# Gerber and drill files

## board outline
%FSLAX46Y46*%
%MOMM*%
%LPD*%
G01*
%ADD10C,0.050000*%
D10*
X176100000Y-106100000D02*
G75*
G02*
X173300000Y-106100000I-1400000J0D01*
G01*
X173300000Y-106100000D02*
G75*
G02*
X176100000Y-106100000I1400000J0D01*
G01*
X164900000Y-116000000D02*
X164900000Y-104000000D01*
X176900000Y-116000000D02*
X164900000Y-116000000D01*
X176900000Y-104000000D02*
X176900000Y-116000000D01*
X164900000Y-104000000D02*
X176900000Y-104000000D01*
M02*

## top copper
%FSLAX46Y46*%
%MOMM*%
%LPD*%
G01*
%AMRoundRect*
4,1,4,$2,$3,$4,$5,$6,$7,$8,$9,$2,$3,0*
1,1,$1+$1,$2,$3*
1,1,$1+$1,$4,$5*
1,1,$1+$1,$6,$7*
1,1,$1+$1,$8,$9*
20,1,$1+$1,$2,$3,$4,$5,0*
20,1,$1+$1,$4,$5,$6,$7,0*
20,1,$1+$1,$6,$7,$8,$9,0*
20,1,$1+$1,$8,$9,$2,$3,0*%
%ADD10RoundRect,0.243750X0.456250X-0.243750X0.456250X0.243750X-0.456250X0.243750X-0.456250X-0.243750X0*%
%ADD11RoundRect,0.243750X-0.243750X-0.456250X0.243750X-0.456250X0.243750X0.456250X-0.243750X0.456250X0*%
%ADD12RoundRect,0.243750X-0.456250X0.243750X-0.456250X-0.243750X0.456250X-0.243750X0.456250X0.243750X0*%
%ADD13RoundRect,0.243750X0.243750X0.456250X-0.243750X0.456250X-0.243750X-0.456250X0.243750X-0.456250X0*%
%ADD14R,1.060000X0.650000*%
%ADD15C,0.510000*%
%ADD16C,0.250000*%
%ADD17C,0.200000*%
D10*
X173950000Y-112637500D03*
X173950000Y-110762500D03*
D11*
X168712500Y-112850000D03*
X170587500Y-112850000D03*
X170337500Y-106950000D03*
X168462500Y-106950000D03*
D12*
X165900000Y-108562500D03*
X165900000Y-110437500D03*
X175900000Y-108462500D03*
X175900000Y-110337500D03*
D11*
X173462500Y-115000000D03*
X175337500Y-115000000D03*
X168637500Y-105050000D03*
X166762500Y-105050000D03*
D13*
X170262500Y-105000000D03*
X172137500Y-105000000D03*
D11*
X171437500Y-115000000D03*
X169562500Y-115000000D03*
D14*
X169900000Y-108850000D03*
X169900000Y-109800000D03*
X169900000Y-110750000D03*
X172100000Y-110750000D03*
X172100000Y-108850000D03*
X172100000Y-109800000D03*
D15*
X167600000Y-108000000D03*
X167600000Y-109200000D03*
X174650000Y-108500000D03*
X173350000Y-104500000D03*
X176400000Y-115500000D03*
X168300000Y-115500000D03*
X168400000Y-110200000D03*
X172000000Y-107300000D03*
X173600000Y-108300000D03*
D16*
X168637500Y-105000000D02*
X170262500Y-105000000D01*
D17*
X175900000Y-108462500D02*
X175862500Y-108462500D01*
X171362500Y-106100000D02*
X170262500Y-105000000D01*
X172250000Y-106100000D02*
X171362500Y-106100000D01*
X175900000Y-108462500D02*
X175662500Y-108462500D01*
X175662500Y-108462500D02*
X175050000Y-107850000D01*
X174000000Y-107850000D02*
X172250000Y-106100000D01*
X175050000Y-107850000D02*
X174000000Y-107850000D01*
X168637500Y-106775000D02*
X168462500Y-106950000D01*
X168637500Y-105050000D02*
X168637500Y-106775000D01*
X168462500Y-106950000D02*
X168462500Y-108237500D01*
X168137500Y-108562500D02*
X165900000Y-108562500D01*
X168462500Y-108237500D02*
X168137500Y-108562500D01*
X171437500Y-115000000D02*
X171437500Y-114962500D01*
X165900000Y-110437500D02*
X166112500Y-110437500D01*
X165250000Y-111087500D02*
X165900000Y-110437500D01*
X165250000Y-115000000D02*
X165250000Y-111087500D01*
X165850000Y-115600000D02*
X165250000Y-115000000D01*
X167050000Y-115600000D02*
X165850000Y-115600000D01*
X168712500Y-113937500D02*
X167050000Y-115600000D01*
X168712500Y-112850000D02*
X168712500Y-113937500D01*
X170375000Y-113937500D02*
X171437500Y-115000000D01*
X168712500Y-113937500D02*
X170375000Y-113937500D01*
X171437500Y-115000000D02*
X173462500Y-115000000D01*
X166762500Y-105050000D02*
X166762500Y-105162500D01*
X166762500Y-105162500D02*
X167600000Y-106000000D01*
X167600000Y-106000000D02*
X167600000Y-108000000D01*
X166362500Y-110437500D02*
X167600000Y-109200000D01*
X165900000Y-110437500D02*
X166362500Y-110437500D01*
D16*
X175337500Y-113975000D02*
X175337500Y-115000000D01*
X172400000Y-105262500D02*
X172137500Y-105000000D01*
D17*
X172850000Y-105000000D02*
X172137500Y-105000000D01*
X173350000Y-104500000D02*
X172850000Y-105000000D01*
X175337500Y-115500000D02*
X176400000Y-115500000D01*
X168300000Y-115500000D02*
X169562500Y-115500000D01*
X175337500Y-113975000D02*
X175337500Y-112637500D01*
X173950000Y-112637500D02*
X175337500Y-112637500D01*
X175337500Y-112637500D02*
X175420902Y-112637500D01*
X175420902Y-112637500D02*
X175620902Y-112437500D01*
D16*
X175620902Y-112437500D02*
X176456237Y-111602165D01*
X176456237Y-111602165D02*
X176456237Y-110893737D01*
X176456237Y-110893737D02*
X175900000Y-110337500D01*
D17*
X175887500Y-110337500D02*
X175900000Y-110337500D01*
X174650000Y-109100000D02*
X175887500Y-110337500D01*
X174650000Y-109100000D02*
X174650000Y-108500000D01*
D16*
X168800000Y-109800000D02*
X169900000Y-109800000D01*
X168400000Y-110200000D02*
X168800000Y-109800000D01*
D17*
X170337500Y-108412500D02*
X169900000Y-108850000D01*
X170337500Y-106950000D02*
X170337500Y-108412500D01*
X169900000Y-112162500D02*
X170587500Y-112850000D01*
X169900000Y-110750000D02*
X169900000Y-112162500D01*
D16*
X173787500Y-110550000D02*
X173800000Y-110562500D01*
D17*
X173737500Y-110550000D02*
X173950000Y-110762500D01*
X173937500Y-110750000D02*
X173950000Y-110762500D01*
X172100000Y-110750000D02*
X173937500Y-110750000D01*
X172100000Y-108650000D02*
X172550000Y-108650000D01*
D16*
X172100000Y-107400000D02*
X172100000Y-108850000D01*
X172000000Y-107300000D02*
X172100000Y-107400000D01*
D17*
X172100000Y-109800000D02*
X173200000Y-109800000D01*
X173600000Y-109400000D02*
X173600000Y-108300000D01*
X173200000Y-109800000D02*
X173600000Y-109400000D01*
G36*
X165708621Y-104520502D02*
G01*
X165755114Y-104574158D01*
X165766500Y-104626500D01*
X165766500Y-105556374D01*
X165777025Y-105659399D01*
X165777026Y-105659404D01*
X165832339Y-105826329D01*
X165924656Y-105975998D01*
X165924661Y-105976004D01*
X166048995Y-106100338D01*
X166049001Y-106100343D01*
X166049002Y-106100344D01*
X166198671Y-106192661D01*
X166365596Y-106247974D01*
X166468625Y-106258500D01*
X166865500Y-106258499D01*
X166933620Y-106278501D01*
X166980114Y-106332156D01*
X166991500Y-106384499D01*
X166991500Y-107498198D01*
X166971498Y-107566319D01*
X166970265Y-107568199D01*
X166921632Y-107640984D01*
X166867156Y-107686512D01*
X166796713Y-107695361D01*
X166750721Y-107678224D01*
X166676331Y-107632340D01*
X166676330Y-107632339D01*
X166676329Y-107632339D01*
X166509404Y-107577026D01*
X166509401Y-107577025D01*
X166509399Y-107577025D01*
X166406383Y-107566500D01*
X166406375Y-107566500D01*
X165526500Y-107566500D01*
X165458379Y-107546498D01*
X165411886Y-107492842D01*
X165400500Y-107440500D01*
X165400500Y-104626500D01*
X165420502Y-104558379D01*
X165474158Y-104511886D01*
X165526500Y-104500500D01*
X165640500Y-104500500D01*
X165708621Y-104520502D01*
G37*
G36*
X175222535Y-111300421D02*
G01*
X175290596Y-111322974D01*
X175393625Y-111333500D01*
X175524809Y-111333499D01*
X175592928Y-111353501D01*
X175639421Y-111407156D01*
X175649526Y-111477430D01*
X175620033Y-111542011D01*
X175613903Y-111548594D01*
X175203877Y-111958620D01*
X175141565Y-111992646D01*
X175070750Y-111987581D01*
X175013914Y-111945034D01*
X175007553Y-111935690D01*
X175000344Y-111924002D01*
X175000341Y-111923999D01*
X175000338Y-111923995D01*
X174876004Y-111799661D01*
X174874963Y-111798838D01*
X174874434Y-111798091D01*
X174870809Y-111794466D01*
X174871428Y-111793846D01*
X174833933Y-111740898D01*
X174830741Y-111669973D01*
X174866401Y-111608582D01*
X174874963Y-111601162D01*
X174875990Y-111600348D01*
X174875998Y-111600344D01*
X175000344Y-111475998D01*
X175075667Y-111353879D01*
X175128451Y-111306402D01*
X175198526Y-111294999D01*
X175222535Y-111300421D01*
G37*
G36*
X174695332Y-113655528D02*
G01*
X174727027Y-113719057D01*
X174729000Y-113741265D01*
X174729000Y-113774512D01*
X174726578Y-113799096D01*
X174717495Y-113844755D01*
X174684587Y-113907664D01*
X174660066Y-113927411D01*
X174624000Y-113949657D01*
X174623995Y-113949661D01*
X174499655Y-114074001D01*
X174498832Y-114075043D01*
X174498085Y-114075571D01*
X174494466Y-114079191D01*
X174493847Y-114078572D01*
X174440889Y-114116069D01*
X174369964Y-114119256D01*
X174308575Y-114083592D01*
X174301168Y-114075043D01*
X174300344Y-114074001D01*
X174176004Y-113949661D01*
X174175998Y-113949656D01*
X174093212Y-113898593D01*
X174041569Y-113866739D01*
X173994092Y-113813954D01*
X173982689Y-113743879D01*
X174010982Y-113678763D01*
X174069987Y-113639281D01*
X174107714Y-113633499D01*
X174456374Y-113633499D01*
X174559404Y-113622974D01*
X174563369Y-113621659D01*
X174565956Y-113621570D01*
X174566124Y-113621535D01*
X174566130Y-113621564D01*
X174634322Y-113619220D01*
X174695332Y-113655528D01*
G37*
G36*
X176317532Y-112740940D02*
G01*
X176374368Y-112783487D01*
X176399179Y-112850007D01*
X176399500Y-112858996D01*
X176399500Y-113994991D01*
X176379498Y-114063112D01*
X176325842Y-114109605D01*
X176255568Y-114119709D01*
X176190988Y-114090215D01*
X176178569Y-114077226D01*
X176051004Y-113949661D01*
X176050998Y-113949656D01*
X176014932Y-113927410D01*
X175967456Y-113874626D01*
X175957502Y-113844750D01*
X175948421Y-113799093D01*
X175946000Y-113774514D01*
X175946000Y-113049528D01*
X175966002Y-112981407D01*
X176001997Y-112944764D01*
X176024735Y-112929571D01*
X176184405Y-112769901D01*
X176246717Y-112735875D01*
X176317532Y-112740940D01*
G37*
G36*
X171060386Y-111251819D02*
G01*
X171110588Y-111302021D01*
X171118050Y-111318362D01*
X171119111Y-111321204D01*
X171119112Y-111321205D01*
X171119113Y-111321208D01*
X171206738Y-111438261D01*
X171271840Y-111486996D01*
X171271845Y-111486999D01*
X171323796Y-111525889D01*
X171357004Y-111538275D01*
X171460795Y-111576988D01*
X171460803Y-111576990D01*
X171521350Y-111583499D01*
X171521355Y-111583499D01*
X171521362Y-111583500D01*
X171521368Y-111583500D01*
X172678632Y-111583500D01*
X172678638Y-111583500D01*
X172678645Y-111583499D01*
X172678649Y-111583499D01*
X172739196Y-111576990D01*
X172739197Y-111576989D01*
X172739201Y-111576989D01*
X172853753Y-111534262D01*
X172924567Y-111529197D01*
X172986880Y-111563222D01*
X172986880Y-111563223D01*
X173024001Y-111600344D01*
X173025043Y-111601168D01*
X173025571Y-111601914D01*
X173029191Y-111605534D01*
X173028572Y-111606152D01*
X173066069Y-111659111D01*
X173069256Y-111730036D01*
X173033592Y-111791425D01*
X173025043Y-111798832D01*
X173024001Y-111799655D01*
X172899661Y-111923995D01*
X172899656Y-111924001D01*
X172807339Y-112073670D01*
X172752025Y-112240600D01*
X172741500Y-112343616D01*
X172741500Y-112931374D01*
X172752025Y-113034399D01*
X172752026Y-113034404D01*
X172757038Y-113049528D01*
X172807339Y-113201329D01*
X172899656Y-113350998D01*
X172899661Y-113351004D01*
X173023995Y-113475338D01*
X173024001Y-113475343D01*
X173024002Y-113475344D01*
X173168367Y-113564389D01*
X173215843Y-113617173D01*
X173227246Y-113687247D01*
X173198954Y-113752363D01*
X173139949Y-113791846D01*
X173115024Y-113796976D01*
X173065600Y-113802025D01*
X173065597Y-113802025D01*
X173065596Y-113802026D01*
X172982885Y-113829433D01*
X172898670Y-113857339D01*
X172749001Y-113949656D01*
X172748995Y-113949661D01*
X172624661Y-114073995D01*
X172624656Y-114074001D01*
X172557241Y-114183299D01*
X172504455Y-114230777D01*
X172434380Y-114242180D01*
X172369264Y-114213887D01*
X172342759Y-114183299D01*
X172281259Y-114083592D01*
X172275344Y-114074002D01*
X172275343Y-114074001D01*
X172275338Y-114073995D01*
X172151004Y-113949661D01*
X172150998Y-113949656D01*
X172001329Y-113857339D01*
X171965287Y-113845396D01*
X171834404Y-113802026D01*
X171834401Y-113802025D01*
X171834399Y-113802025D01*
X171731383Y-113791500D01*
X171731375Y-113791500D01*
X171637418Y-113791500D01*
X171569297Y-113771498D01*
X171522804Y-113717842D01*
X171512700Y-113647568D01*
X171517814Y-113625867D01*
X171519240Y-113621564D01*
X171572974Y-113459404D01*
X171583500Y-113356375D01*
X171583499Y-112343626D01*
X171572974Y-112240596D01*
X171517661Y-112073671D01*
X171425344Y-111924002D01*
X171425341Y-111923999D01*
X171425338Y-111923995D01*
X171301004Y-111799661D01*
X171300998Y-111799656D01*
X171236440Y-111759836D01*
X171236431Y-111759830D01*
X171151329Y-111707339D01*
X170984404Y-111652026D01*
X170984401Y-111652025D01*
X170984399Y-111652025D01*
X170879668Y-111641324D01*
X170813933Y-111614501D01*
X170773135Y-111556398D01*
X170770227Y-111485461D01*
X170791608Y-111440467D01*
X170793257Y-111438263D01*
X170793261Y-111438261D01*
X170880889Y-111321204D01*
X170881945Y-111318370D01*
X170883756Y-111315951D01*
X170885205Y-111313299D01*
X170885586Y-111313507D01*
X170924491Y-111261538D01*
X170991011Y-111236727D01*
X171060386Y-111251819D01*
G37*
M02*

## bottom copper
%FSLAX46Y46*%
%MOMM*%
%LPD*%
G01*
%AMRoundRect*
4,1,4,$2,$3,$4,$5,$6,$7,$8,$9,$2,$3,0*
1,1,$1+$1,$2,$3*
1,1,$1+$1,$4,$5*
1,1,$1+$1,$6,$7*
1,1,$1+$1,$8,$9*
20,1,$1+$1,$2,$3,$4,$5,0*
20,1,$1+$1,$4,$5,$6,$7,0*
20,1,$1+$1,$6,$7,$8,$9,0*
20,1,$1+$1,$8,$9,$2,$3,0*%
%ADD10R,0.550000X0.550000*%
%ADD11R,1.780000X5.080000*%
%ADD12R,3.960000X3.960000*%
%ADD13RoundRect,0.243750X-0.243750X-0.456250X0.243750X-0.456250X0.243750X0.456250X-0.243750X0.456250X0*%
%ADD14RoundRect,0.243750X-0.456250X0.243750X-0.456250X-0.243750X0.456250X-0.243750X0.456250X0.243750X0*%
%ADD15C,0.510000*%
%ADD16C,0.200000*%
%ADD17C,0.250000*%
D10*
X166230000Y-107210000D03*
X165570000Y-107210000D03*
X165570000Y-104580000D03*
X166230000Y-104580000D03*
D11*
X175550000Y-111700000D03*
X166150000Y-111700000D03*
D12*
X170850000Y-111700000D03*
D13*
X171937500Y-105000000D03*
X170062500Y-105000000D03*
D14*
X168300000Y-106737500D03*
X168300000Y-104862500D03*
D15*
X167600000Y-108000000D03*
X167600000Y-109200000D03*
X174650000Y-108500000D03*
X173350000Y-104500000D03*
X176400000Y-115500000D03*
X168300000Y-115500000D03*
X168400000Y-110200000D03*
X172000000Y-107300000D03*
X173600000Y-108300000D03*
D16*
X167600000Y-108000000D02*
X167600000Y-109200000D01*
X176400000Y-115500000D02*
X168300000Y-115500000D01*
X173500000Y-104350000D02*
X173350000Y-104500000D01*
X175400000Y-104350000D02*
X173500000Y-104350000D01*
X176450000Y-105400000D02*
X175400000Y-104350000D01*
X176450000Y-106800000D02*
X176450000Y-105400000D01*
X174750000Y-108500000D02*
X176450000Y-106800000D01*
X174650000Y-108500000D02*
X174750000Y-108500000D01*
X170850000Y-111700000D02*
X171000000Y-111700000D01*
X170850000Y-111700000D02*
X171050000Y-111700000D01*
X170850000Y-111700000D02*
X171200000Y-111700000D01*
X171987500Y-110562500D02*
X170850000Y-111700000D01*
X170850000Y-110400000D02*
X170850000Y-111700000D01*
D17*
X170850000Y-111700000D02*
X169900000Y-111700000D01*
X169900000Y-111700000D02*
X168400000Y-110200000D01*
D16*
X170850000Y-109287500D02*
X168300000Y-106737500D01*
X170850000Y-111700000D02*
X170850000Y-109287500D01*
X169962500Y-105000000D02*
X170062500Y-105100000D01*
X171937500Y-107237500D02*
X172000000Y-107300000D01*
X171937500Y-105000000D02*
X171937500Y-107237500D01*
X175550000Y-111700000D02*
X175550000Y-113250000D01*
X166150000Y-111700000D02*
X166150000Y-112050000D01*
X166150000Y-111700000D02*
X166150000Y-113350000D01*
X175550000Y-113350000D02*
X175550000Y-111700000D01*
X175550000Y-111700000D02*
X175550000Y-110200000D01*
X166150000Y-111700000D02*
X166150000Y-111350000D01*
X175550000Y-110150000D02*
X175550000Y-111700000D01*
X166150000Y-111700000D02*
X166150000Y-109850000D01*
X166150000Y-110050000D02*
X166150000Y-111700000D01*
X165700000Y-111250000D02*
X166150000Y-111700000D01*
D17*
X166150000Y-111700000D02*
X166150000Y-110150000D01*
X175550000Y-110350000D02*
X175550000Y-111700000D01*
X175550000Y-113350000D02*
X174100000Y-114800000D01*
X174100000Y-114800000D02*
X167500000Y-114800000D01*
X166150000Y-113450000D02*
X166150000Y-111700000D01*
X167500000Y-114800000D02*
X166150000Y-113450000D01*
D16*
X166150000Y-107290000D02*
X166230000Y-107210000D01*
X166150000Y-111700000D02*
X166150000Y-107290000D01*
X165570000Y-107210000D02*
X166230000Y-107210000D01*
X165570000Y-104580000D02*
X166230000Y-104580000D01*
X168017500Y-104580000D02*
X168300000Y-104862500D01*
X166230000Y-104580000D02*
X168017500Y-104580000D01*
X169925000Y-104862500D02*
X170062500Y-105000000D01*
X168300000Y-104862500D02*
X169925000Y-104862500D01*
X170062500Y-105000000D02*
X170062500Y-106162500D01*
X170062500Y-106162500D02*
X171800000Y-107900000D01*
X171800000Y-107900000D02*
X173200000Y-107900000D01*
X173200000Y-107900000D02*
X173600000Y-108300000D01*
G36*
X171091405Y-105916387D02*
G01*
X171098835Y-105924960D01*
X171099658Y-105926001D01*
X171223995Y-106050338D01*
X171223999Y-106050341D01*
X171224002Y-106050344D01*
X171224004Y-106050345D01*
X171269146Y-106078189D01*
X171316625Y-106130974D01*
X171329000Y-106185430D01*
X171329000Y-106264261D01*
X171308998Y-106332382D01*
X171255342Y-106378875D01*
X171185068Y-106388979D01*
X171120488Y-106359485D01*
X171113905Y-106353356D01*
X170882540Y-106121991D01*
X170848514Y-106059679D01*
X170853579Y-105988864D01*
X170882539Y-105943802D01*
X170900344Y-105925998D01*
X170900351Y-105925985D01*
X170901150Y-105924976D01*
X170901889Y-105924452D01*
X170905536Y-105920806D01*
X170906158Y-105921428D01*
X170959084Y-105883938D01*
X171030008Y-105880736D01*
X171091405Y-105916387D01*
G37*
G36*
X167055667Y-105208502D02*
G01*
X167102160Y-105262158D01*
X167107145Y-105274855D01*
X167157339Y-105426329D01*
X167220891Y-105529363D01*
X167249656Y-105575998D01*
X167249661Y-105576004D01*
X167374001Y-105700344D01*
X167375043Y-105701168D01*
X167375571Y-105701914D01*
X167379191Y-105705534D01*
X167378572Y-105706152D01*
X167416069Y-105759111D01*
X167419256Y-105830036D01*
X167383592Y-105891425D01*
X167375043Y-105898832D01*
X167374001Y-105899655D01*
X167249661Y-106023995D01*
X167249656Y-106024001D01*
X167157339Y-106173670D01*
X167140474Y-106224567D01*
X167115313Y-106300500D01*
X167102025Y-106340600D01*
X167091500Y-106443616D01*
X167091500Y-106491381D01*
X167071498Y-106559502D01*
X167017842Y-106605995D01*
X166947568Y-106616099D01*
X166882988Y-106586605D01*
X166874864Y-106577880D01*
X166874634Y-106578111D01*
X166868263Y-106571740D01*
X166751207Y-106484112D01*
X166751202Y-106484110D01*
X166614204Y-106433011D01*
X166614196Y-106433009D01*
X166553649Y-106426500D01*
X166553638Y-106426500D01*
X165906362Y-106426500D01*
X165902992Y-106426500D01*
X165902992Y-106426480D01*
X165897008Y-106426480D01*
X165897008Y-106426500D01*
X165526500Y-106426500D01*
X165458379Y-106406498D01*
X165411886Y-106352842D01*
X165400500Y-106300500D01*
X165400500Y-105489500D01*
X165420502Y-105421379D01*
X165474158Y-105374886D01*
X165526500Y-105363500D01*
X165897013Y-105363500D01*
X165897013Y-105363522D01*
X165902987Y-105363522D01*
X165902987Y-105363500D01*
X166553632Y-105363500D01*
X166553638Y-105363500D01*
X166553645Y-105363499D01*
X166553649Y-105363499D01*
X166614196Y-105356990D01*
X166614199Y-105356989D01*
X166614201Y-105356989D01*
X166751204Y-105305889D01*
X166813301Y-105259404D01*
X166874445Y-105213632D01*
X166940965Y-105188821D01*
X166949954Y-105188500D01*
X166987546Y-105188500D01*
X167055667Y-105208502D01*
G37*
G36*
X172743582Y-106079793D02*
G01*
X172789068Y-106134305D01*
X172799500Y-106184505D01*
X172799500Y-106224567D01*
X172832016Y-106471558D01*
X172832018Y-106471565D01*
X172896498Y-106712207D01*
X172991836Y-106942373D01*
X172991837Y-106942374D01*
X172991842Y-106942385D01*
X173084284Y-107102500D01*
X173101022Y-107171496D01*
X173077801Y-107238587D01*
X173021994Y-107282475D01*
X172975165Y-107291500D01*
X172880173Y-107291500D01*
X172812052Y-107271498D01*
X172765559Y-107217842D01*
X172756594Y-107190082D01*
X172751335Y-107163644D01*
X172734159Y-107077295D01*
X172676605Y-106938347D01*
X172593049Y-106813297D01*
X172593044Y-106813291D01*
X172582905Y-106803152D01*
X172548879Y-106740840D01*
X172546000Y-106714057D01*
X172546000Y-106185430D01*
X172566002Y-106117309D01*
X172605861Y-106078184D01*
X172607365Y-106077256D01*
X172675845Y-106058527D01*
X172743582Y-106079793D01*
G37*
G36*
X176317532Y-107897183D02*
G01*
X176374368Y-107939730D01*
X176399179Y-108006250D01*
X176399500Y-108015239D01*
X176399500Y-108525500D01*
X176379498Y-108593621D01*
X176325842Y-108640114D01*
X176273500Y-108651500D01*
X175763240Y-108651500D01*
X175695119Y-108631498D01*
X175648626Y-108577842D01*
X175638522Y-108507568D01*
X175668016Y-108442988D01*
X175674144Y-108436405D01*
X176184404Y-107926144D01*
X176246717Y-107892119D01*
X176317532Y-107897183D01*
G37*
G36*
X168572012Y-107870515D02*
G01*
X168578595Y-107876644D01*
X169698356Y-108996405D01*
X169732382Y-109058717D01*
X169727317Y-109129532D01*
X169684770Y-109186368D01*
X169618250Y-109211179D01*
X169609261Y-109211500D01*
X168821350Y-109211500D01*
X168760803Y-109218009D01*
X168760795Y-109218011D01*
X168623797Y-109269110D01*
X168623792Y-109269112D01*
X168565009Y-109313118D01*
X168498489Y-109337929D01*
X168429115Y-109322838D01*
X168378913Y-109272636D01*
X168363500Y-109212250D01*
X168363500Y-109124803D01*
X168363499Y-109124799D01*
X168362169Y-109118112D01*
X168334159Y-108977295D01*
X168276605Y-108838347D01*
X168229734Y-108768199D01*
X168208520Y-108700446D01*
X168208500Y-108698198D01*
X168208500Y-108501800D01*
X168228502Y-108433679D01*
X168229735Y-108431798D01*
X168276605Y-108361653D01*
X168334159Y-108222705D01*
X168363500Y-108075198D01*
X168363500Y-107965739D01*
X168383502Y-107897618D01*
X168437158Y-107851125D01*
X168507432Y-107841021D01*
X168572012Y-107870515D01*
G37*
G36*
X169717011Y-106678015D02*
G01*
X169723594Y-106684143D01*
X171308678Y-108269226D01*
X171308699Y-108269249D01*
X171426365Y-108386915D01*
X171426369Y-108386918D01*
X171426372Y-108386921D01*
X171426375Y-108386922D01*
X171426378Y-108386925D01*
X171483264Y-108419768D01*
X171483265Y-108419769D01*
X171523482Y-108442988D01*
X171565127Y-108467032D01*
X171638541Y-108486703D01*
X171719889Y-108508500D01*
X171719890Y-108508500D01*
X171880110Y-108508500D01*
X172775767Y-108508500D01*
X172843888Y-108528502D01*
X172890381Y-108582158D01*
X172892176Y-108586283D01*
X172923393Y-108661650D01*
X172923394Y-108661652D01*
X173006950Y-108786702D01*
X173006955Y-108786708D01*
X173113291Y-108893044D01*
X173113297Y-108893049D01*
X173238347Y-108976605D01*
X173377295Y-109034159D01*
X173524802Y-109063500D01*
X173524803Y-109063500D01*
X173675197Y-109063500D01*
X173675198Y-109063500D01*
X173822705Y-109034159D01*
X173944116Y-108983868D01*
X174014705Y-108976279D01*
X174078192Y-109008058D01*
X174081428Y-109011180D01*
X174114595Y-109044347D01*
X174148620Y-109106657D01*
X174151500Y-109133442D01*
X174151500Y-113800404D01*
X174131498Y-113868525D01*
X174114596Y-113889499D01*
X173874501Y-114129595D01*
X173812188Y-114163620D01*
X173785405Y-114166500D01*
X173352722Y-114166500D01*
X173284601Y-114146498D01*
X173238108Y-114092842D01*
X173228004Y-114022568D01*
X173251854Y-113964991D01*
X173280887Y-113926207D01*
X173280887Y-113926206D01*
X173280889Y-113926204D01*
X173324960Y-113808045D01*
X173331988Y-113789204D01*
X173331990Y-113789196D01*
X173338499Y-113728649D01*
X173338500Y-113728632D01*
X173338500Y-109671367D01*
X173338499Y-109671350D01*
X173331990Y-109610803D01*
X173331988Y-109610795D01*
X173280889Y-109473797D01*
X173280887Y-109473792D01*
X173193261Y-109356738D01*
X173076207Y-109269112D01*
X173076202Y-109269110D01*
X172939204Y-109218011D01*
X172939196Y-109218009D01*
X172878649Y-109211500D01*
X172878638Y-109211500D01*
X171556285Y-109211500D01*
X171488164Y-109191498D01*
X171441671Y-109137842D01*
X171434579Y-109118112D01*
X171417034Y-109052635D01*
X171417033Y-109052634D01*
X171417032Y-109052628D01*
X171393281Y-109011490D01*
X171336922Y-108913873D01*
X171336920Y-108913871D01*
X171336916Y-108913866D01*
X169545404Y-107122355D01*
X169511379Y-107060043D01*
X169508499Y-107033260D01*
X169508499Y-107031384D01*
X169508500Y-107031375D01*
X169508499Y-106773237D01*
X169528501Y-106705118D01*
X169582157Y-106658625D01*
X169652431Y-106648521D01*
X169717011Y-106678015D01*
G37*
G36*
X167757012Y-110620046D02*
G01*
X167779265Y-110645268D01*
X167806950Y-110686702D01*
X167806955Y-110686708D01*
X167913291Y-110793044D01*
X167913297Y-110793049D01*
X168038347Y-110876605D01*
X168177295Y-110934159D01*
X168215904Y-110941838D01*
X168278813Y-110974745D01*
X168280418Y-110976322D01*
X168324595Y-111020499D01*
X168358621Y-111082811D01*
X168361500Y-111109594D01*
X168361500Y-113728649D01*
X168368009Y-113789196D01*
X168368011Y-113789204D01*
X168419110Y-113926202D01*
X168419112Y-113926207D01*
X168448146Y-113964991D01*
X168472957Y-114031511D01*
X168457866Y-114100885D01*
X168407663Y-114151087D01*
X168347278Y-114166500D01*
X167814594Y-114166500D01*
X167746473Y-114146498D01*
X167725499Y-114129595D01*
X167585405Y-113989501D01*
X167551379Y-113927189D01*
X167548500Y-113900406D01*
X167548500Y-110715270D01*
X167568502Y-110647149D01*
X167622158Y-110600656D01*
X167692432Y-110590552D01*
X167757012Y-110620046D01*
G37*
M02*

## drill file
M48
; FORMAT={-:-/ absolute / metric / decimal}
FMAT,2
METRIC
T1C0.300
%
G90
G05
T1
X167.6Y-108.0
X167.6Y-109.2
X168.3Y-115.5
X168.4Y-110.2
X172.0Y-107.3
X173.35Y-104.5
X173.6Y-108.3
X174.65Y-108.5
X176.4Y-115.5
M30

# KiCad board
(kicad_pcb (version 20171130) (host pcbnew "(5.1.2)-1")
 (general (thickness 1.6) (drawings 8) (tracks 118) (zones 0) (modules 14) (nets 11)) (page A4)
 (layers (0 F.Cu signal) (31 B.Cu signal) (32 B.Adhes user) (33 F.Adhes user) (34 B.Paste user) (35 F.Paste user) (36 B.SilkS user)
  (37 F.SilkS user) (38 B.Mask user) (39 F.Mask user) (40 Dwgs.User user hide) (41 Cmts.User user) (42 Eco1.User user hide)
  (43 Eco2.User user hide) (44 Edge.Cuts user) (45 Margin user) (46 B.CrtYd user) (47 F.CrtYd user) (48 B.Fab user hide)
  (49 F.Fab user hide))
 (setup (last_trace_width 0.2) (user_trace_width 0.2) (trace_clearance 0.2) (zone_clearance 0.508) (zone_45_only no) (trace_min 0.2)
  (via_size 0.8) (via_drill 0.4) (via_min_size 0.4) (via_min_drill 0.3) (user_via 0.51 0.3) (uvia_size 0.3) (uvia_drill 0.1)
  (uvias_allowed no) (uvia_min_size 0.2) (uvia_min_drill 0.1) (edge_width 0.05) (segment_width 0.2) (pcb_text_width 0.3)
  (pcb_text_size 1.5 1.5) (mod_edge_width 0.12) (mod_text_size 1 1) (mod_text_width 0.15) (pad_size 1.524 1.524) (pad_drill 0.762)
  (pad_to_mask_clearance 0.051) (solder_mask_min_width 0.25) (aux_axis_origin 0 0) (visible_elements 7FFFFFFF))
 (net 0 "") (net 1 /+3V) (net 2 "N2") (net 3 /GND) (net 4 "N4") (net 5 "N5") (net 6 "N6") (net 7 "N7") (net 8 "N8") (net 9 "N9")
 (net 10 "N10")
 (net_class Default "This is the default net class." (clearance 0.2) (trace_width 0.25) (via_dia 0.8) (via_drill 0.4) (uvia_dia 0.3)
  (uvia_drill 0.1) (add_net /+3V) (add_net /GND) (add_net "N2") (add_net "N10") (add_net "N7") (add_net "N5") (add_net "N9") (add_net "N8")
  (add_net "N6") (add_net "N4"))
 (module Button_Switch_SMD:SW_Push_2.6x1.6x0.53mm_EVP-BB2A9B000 (layer B.Cu) (at 165.9 105.9 90)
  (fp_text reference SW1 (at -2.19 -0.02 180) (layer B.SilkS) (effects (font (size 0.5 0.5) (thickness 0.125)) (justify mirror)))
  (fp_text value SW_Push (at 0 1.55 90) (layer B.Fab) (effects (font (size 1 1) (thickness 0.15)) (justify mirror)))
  (pad 1 smd rect (at -1.31 0.33 90) (size 0.55 0.55) (layers B.Cu B.Paste B.Mask) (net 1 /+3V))
  (pad 1 smd rect (at -1.31 -0.33 90) (size 0.55 0.55) (layers B.Cu B.Paste B.Mask) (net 1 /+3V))
  (pad 2 smd rect (at 1.32 -0.33 90) (size 0.55 0.55) (layers B.Cu B.Paste B.Mask) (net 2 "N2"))
  (pad 2 smd rect (at 1.32 0.33 90) (size 0.55 0.55) (layers B.Cu B.Paste B.Mask) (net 2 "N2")))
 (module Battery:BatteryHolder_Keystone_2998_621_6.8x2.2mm (layer B.Cu) (at 170.85 111.7)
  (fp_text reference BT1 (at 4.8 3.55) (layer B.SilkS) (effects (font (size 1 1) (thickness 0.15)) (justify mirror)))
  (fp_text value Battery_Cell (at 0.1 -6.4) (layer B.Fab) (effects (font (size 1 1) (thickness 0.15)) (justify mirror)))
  (pad 1 smd rect (at 4.7 0) (size 1.78 5.08) (layers B.Cu B.Paste B.Mask) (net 1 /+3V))
  (pad 1 smd rect (at -4.7 0) (size 1.78 5.08) (layers B.Cu B.Paste B.Mask) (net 1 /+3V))
  (pad 2 smd rect (at 0 0) (size 3.96 3.96) (layers B.Cu B.Paste B.Mask) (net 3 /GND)))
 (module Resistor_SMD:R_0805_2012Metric (layer B.Cu) (at 171 105)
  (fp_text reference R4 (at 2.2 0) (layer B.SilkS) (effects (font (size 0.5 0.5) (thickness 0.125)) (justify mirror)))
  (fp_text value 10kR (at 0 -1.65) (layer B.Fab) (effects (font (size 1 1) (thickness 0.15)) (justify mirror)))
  (pad 2 smd roundrect (at 0.9375 0) (size 0.975 1.4) (layers B.Cu B.Paste B.Mask) (roundrect_rratio 0.25) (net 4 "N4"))
  (pad 1 smd roundrect (at -0.9375 0) (size 0.975 1.4) (layers B.Cu B.Paste B.Mask) (roundrect_rratio 0.25) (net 2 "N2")))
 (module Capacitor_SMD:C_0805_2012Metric (layer B.Cu) (at 168.3 105.8 270)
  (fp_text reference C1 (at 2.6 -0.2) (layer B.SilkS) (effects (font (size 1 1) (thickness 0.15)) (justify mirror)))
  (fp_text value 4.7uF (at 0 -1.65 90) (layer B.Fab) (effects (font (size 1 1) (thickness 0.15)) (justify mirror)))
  (pad 2 smd roundrect (at 0.9375 0 270) (size 0.975 1.4) (layers B.Cu B.Paste B.Mask) (roundrect_rratio 0.25) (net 3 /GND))
  (pad 1 smd roundrect (at -0.9375 0 270) (size 0.975 1.4) (layers B.Cu B.Paste B.Mask) (roundrect_rratio 0.25) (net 2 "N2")))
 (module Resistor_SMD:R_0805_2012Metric (layer F.Cu) (at 173.95 111.7 90)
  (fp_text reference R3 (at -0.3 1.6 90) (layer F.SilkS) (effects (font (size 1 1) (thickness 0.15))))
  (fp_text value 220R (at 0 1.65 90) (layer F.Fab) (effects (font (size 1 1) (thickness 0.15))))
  (pad 1 smd roundrect (at -0.9375 0 90) (size 0.975 1.4) (layers F.Cu F.Paste F.Mask) (roundrect_rratio 0.25) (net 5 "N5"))
  (pad 2 smd roundrect (at 0.9375 0 90) (size 0.975 1.4) (layers F.Cu F.Paste F.Mask) (roundrect_rratio 0.25) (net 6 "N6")))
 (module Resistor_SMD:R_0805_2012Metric (layer F.Cu) (at 169.65 112.85)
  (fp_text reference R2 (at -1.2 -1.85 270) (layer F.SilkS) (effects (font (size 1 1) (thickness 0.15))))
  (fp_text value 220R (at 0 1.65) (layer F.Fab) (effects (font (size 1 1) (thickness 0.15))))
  (pad 1 smd roundrect (at -0.9375 0) (size 0.975 1.4) (layers F.Cu F.Paste F.Mask) (roundrect_rratio 0.25) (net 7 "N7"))
  (pad 2 smd roundrect (at 0.9375 0) (size 0.975 1.4) (layers F.Cu F.Paste F.Mask) (roundrect_rratio 0.25) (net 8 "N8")))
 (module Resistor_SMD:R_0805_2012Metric (layer F.Cu) (at 169.4 106.95)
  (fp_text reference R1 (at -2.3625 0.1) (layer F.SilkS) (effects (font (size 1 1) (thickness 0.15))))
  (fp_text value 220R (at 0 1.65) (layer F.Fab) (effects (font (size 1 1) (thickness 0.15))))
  (pad 2 smd roundrect (at 0.9375 0) (size 0.975 1.4) (layers F.Cu F.Paste F.Mask) (roundrect_rratio 0.25) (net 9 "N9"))
  (pad 1 smd roundrect (at -0.9375 0) (size 0.975 1.4) (layers F.Cu F.Paste F.Mask) (roundrect_rratio 0.25) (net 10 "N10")))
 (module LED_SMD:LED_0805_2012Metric (layer F.Cu) (at 165.9 109.5 270)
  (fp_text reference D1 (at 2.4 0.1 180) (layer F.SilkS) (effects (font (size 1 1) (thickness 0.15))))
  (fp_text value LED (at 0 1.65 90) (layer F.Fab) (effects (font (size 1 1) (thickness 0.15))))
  (pad 1 smd roundrect (at -0.9375 0 270) (size 0.975 1.4) (layers F.Cu F.Paste F.Mask) (roundrect_rratio 0.25) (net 10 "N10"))
  (pad 2 smd roundrect (at 0.9375 0 270) (size 0.975 1.4) (layers F.Cu F.Paste F.Mask) (roundrect_rratio 0.25) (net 7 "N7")))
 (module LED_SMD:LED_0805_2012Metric (layer F.Cu) (at 175.9 109.4 270)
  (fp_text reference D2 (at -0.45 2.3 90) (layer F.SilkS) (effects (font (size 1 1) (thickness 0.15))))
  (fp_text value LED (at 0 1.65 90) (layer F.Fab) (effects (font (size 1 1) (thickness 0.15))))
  (pad 1 smd roundrect (at -0.9375 0 270) (size 0.975 1.4) (layers F.Cu F.Paste F.Mask) (roundrect_rratio 0.25) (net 10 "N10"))
  (pad 2 smd roundrect (at 0.9375 0 270) (size 0.975 1.4) (layers F.Cu F.Paste F.Mask) (roundrect_rratio 0.25) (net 5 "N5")))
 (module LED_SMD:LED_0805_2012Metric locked (layer F.Cu) (at 174.4 115)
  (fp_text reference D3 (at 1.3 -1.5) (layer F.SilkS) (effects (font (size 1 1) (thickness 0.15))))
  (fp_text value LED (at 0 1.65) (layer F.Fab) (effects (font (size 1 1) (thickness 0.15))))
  (pad 1 smd roundrect (at -0.9375 0) (size 0.975 1.4) (layers F.Cu F.Paste F.Mask) (roundrect_rratio 0.25) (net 7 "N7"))
  (pad 2 smd roundrect (at 0.9375 0) (size 0.975 1.4) (layers F.Cu F.Paste F.Mask) (roundrect_rratio 0.25) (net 5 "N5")))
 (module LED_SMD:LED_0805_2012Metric (layer F.Cu) (at 167.7 105.05)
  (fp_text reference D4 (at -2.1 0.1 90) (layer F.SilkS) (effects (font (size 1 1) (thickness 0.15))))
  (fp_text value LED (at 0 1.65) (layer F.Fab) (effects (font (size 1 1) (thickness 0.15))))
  (pad 2 smd roundrect (at 0.9375 0) (size 0.975 1.4) (layers F.Cu F.Paste F.Mask) (roundrect_rratio 0.25) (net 10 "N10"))
  (pad 1 smd roundrect (at -0.9375 0) (size 0.975 1.4) (layers F.Cu F.Paste F.Mask) (roundrect_rratio 0.25) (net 7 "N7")))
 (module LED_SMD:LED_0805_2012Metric (layer F.Cu) (at 171.2 105 180)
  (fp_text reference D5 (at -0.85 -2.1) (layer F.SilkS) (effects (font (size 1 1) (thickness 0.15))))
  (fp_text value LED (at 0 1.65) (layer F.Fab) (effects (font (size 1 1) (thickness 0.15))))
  (pad 2 smd roundrect (at 0.9375 0 180) (size 0.975 1.4) (layers F.Cu F.Paste F.Mask) (roundrect_rratio 0.25) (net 10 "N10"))
  (pad 1 smd roundrect (at -0.9375 0 180) (size 0.975 1.4) (layers F.Cu F.Paste F.Mask) (roundrect_rratio 0.25) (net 5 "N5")))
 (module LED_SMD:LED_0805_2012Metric (layer F.Cu) (at 170.5 115)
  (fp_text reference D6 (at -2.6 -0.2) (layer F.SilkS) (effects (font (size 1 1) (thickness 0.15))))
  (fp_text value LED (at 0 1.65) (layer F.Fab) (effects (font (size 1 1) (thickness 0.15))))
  (pad 2 smd roundrect (at 0.9375 0) (size 0.975 1.4) (layers F.Cu F.Paste F.Mask) (roundrect_rratio 0.25) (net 7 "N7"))
  (pad 1 smd roundrect (at -0.9375 0) (size 0.975 1.4) (layers F.Cu F.Paste F.Mask) (roundrect_rratio 0.25) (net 5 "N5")))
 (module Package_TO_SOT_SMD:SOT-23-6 (layer F.Cu) (at 171 109.8)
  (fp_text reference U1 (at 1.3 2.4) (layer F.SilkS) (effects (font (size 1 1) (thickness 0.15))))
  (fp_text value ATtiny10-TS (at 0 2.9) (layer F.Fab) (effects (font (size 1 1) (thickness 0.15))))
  (pad 1 smd rect (at -1.1 -0.95) (size 1.06 0.65) (layers F.Cu F.Paste F.Mask) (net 9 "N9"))
  (pad 2 smd rect (at -1.1 0) (size 1.06 0.65) (layers F.Cu F.Paste F.Mask) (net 3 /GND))
  (pad 3 smd rect (at -1.1 0.95) (size 1.06 0.65) (layers F.Cu F.Paste F.Mask) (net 8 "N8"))
  (pad 4 smd rect (at 1.1 0.95) (size 1.06 0.65) (layers F.Cu F.Paste F.Mask) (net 6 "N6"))
  (pad 6 smd rect (at 1.1 -0.95) (size 1.06 0.65) (layers F.Cu F.Paste F.Mask) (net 4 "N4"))
  (pad 5 smd rect (at 1.1 0) (size 1.06 0.65) (layers F.Cu F.Paste F.Mask) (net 2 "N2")))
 (gr_circle (center 174.7 106.1) (end 176.1 106.1) (layer Edge.Cuts) (width 0.05))
 (gr_line (start 164.9 116) (end 164.9 104) (layer Edge.Cuts) (width 0.05))
 (gr_line (start 176.9 116) (end 164.9 116) (layer Edge.Cuts) (width 0.05))
 (gr_line (start 176.9 104) (end 176.9 116) (layer Edge.Cuts) (width 0.05))
 (gr_line (start 164.9 104) (end 176.9 104) (layer Edge.Cuts) (width 0.05))
 (segment (start 168.6375 105) (end 170.2625 105) (width 0.25) (layer F.Cu) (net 10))
 (segment (start 175.9 108.4625) (end 175.8625 108.4625) (width 0.2) (layer F.Cu) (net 10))
 (segment (start 171.3625 106.1) (end 170.2625 105) (width 0.2) (layer F.Cu) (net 10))
 (segment (start 172.25 106.1) (end 171.3625 106.1) (width 0.2) (layer F.Cu) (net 10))
 (segment (start 175.9 108.4625) (end 175.6625 108.4625) (width 0.2) (layer F.Cu) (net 10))
 (segment (start 175.6625 108.4625) (end 175.05 107.85) (width 0.2) (layer F.Cu) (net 10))
 (segment (start 174 107.85) (end 172.25 106.1) (width 0.2) (layer F.Cu) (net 10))
 (segment (start 175.05 107.85) (end 174 107.85) (width 0.2) (layer F.Cu) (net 10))
 (segment (start 168.6375 106.775) (end 168.4625 106.95) (width 0.2) (layer F.Cu) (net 10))
 (segment (start 168.6375 105.05) (end 168.6375 106.775) (width 0.2) (layer F.Cu) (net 10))
 (segment (start 168.4625 106.95) (end 168.4625 108.2375) (width 0.2) (layer F.Cu) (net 10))
 (segment (start 168.1375 108.5625) (end 165.9 108.5625) (width 0.2) (layer F.Cu) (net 10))
 (segment (start 168.4625 108.2375) (end 168.1375 108.5625) (width 0.2) (layer F.Cu) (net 10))
 (segment (start 171.4375 115) (end 171.4375 114.9625) (width 0.2) (layer F.Cu) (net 7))
 (segment (start 165.9 110.4375) (end 166.1125 110.4375) (width 0.2) (layer F.Cu) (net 7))
 (segment (start 165.25 111.0875) (end 165.9 110.4375) (width 0.2) (layer F.Cu) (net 7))
 (segment (start 165.25 115) (end 165.25 111.0875) (width 0.2) (layer F.Cu) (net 7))
 (segment (start 165.85 115.6) (end 165.25 115) (width 0.2) (layer F.Cu) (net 7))
 (segment (start 167.05 115.6) (end 165.85 115.6) (width 0.2) (layer F.Cu) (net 7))
 (segment (start 168.7125 113.9375) (end 167.05 115.6) (width 0.2) (layer F.Cu) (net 7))
 (segment (start 168.7125 112.85) (end 168.7125 113.9375) (width 0.2) (layer F.Cu) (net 7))
 (segment (start 170.375 113.9375) (end 171.4375 115) (width 0.2) (layer F.Cu) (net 7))
 (segment (start 168.7125 113.9375) (end 170.375 113.9375) (width 0.2) (layer F.Cu) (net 7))
 (segment (start 171.4375 115) (end 173.4625 115) (width 0.2) (layer F.Cu) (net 7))
 (segment (start 166.7625 105.05) (end 166.7625 105.1625) (width 0.2) (layer F.Cu) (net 7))
 (via (at 167.6 108) (size 0.51) (drill 0.3) (layers F.Cu B.Cu) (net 7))
 (segment (start 166.7625 105.1625) (end 167.6 106) (width 0.2) (layer F.Cu) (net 7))
 (segment (start 167.6 106) (end 167.6 108) (width 0.2) (layer F.Cu) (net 7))
 (via (at 167.6 109.2) (size 0.51) (drill 0.3) (layers F.Cu B.Cu) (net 7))
 (segment (start 167.6 108) (end 167.6 109.2) (width 0.2) (layer B.Cu) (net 7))
 (segment (start 166.3625 110.4375) (end 167.6 109.2) (width 0.2) (layer F.Cu) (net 7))
 (segment (start 165.9 110.4375) (end 166.3625 110.4375) (width 0.2) (layer F.Cu) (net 7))
 (segment (start 175.3375 113.975) (end 175.3375 115) (width 0.25) (layer F.Cu) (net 5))
 (via (at 174.65 108.5) (size 0.51) (drill 0.3) (layers F.Cu B.Cu) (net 5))
 (segment (start 172.4 105.2625) (end 172.1375 105) (width 0.25) (layer F.Cu) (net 5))
 (via (at 173.35 104.5) (size 0.51) (drill 0.3) (layers F.Cu B.Cu) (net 5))
 (segment (start 172.85 105) (end 172.1375 105) (width 0.2) (layer F.Cu) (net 5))
 (segment (start 173.35 104.5) (end 172.85 105) (width 0.2) (layer F.Cu) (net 5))
 (via (at 176.4 115.5) (size 0.51) (drill 0.3) (layers F.Cu B.Cu) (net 5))
 (segment (start 175.3375 115.5) (end 176.4 115.5) (width 0.2) (layer F.Cu) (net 5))
 (via (at 168.3 115.5) (size 0.51) (drill 0.3) (layers F.Cu B.Cu) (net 5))
 (segment (start 176.4 115.5) (end 168.3 115.5) (width 0.2) (layer B.Cu) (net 5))
 (segment (start 168.3 115.5) (end 169.5625 115.5) (width 0.2) (layer F.Cu) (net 5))
 (segment (start 175.3375 113.975) (end 175.3375 112.6375) (width 0.2) (layer F.Cu) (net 5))
 (segment (start 173.95 112.6375) (end 175.3375 112.6375) (width 0.2) (layer F.Cu) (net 5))
 (segment (start 175.3375 112.6375) (end 175.420902 112.6375) (width 0.2) (layer F.Cu) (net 5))
 (segment (start 175.420902 112.6375) (end 175.620902 112.4375) (width 0.2) (layer F.Cu) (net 5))
 (segment (start 175.620902 112.4375) (end 176.456237 111.602165) (width 0.25) (layer F.Cu) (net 5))
 (segment (start 176.456237 111.602165) (end 176.456237 110.893737) (width 0.25) (layer F.Cu) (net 5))
 (segment (start 176.456237 110.893737) (end 175.9 110.3375) (width 0.25) (layer F.Cu) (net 5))
 (segment (start 173.5 104.35) (end 173.35 104.5) (width 0.2) (layer B.Cu) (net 5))
 (segment (start 175.4 104.35) (end 173.5 104.35) (width 0.2) (layer B.Cu) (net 5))
 (segment (start 176.45 105.4) (end 175.4 104.35) (width 0.2) (layer B.Cu) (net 5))
 (segment (start 176.45 106.8) (end 176.45 105.4) (width 0.2) (layer B.Cu) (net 5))
 (segment (start 175.8875 110.3375) (end 175.9 110.3375) (width 0.2) (layer F.Cu) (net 5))
 (segment (start 174.65 109.1) (end 175.8875 110.3375) (width 0.2) (layer F.Cu) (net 5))
 (segment (start 174.65 109.1) (end 174.65 108.5) (width 0.2) (layer F.Cu) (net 5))
 (segment (start 174.75 108.5) (end 176.45 106.8) (width 0.2) (layer B.Cu) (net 5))
 (segment (start 174.65 108.5) (end 174.75 108.5) (width 0.2) (layer B.Cu) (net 5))
 (segment (start 170.85 111.7) (end 171 111.7) (width 0.2) (layer B.Cu) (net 3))
 (segment (start 170.85 111.7) (end 171.05 111.7) (width 0.2) (layer B.Cu) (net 3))
 (segment (start 170.85 111.7) (end 171.2 111.7) (width 0.2) (layer B.Cu) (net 3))
 (segment (start 171.9875 110.5625) (end 170.85 111.7) (width 0.2) (layer B.Cu) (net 3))
 (segment (start 170.85 110.4) (end 170.85 111.7) (width 0.2) (layer B.Cu) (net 3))
 (via (at 168.4 110.2) (size 0.51) (drill 0.3) (layers F.Cu B.Cu) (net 3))
 (segment (start 170.85 111.7) (end 169.9 111.7) (width 0.25) (layer B.Cu) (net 3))
 (segment (start 169.9 111.7) (end 168.4 110.2) (width 0.25) (layer B.Cu) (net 3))
 (segment (start 168.8 109.8) (end 169.9 109.8) (width 0.25) (layer F.Cu) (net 3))
 (segment (start 168.4 110.2) (end 168.8 109.8) (width 0.25) (layer F.Cu) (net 3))
 (segment (start 170.85 109.2875) (end 168.3 106.7375) (width 0.2) (layer B.Cu) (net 3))
 (segment (start 170.85 111.7) (end 170.85 109.2875) (width 0.2) (layer B.Cu) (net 3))
 (segment (start 170.3375 108.4125) (end 169.9 108.85) (width 0.2) (layer F.Cu) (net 9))
 (segment (start 170.3375 106.95) (end 170.3375 108.4125) (width 0.2) (layer F.Cu) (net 9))
 (segment (start 169.9 112.1625) (end 170.5875 112.85) (width 0.2) (layer F.Cu) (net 8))
 (segment (start 169.9 110.75) (end 169.9 112.1625) (width 0.2) (layer F.Cu) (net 8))
 (segment (start 173.7875 110.55) (end 173.8 110.5625) (width 0.25) (layer F.Cu) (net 6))
 (segment (start 173.7375 110.55) (end 173.95 110.7625) (width 0.2) (layer F.Cu) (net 6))
 (segment (start 173.9375 110.75) (end 173.95 110.7625) (width 0.2) (layer F.Cu) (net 6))
 (segment (start 172.1 110.75) (end 173.9375 110.75) (width 0.2) (layer F.Cu) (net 6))
 (segment (start 172.1 108.65) (end 172.55 108.65) (width 0.2) (layer F.Cu) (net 4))
 (segment (start 169.9625 105) (end 170.0625 105.1) (width 0.2) (layer B.Cu) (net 2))
 (via (at 172 107.3) (size 0.51) (drill 0.3) (layers F.Cu B.Cu) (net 4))
 (segment (start 172.1 107.4) (end 172.1 108.85) (width 0.25) (layer F.Cu) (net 4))
 (segment (start 172 107.3) (end 172.1 107.4) (width 0.25) (layer F.Cu) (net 4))
 (segment (start 171.9375 107.2375) (end 172 107.3) (width 0.2) (layer B.Cu) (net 4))
 (segment (start 171.9375 105) (end 171.9375 107.2375) (width 0.2) (layer B.Cu) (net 4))
 (segment (start 175.55 111.7) (end 175.55 113.25) (width 0.2) (layer B.Cu) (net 1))
 (segment (start 166.15 111.7) (end 166.15 112.05) (width 0.2) (layer B.Cu) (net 1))
 (segment (start 166.15 111.7) (end 166.15 113.35) (width 0.2) (layer B.Cu) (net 1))
 (segment (start 175.55 113.35) (end 175.55 111.7) (width 0.2) (layer B.Cu) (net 1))
 (segment (start 175.55 111.7) (end 175.55 110.2) (width 0.2) (layer B.Cu) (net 1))
 (segment (start 166.15 111.7) (end 166.15 111.35) (width 0.2) (layer B.Cu) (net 1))
 (segment (start 175.55 110.15) (end 175.55 111.7) (width 0.2) (layer B.Cu) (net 1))
 (segment (start 166.15 111.7) (end 166.15 109.85) (width 0.2) (layer B.Cu) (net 1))
 (segment (start 166.15 110.05) (end 166.15 111.7) (width 0.2) (layer B.Cu) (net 1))
 (segment (start 165.7 111.25) (end 166.15 111.7) (width 0.2) (layer B.Cu) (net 1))
 (segment (start 166.15 111.7) (end 166.15 110.15) (width 0.25) (layer B.Cu) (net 1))
 (segment (start 175.55 110.35) (end 175.55 111.7) (width 0.25) (layer B.Cu) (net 1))
 (segment (start 175.55 113.35) (end 174.1 114.8) (width 0.25) (layer B.Cu) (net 1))
 (segment (start 174.1 114.8) (end 167.5 114.8) (width 0.25) (layer B.Cu) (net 1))
 (segment (start 166.15 113.45) (end 166.15 111.7) (width 0.25) (layer B.Cu) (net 1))
 (segment (start 167.5 114.8) (end 166.15 113.45) (width 0.25) (layer B.Cu) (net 1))
 (segment (start 166.15 107.29) (end 166.23 107.21) (width 0.2) (layer B.Cu) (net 1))
 (segment (start 166.15 111.7) (end 166.15 107.29) (width 0.2) (layer B.Cu) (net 1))
 (segment (start 165.57 107.21) (end 166.23 107.21) (width 0.2) (layer B.Cu) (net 1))
 (segment (start 165.57 104.58) (end 166.23 104.58) (width 0.2) (layer B.Cu) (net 2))
 (segment (start 168.0175 104.58) (end 168.3 104.8625) (width 0.2) (layer B.Cu) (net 2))
 (segment (start 166.23 104.58) (end 168.0175 104.58) (width 0.2) (layer B.Cu) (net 2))
 (segment (start 169.925 104.8625) (end 170.0625 105) (width 0.2) (layer B.Cu) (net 2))
 (segment (start 168.3 104.8625) (end 169.925 104.8625) (width 0.2) (layer B.Cu) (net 2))
 (segment (start 170.0625 105) (end 170.0625 106.1625) (width 0.2) (layer B.Cu) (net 2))
 (segment (start 170.0625 106.1625) (end 171.8 107.9) (width 0.2) (layer B.Cu) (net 2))
 (via (at 173.6 108.3) (size 0.51) (drill 0.3) (layers F.Cu B.Cu) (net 2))
 (segment (start 171.8 107.9) (end 173.2 107.9) (width 0.2) (layer B.Cu) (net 2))
 (segment (start 173.2 107.9) (end 173.6 108.3) (width 0.2) (layer B.Cu) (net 2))
 (segment (start 172.1 109.8) (end 173.2 109.8) (width 0.2) (layer F.Cu) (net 2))
 (segment (start 173.6 109.4) (end 173.6 108.3) (width 0.2) (layer F.Cu) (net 2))
 (segment (start 173.2 109.8) (end 173.6 109.4) (width 0.2) (layer F.Cu) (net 2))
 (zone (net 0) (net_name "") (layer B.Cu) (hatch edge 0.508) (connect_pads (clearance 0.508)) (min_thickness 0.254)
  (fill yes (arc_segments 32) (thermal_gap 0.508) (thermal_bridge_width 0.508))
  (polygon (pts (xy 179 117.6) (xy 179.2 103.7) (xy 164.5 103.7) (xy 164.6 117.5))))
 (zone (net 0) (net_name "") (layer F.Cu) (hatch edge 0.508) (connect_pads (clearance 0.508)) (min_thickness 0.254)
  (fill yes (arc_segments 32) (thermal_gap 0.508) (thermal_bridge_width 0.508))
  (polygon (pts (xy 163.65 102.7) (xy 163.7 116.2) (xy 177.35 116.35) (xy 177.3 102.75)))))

